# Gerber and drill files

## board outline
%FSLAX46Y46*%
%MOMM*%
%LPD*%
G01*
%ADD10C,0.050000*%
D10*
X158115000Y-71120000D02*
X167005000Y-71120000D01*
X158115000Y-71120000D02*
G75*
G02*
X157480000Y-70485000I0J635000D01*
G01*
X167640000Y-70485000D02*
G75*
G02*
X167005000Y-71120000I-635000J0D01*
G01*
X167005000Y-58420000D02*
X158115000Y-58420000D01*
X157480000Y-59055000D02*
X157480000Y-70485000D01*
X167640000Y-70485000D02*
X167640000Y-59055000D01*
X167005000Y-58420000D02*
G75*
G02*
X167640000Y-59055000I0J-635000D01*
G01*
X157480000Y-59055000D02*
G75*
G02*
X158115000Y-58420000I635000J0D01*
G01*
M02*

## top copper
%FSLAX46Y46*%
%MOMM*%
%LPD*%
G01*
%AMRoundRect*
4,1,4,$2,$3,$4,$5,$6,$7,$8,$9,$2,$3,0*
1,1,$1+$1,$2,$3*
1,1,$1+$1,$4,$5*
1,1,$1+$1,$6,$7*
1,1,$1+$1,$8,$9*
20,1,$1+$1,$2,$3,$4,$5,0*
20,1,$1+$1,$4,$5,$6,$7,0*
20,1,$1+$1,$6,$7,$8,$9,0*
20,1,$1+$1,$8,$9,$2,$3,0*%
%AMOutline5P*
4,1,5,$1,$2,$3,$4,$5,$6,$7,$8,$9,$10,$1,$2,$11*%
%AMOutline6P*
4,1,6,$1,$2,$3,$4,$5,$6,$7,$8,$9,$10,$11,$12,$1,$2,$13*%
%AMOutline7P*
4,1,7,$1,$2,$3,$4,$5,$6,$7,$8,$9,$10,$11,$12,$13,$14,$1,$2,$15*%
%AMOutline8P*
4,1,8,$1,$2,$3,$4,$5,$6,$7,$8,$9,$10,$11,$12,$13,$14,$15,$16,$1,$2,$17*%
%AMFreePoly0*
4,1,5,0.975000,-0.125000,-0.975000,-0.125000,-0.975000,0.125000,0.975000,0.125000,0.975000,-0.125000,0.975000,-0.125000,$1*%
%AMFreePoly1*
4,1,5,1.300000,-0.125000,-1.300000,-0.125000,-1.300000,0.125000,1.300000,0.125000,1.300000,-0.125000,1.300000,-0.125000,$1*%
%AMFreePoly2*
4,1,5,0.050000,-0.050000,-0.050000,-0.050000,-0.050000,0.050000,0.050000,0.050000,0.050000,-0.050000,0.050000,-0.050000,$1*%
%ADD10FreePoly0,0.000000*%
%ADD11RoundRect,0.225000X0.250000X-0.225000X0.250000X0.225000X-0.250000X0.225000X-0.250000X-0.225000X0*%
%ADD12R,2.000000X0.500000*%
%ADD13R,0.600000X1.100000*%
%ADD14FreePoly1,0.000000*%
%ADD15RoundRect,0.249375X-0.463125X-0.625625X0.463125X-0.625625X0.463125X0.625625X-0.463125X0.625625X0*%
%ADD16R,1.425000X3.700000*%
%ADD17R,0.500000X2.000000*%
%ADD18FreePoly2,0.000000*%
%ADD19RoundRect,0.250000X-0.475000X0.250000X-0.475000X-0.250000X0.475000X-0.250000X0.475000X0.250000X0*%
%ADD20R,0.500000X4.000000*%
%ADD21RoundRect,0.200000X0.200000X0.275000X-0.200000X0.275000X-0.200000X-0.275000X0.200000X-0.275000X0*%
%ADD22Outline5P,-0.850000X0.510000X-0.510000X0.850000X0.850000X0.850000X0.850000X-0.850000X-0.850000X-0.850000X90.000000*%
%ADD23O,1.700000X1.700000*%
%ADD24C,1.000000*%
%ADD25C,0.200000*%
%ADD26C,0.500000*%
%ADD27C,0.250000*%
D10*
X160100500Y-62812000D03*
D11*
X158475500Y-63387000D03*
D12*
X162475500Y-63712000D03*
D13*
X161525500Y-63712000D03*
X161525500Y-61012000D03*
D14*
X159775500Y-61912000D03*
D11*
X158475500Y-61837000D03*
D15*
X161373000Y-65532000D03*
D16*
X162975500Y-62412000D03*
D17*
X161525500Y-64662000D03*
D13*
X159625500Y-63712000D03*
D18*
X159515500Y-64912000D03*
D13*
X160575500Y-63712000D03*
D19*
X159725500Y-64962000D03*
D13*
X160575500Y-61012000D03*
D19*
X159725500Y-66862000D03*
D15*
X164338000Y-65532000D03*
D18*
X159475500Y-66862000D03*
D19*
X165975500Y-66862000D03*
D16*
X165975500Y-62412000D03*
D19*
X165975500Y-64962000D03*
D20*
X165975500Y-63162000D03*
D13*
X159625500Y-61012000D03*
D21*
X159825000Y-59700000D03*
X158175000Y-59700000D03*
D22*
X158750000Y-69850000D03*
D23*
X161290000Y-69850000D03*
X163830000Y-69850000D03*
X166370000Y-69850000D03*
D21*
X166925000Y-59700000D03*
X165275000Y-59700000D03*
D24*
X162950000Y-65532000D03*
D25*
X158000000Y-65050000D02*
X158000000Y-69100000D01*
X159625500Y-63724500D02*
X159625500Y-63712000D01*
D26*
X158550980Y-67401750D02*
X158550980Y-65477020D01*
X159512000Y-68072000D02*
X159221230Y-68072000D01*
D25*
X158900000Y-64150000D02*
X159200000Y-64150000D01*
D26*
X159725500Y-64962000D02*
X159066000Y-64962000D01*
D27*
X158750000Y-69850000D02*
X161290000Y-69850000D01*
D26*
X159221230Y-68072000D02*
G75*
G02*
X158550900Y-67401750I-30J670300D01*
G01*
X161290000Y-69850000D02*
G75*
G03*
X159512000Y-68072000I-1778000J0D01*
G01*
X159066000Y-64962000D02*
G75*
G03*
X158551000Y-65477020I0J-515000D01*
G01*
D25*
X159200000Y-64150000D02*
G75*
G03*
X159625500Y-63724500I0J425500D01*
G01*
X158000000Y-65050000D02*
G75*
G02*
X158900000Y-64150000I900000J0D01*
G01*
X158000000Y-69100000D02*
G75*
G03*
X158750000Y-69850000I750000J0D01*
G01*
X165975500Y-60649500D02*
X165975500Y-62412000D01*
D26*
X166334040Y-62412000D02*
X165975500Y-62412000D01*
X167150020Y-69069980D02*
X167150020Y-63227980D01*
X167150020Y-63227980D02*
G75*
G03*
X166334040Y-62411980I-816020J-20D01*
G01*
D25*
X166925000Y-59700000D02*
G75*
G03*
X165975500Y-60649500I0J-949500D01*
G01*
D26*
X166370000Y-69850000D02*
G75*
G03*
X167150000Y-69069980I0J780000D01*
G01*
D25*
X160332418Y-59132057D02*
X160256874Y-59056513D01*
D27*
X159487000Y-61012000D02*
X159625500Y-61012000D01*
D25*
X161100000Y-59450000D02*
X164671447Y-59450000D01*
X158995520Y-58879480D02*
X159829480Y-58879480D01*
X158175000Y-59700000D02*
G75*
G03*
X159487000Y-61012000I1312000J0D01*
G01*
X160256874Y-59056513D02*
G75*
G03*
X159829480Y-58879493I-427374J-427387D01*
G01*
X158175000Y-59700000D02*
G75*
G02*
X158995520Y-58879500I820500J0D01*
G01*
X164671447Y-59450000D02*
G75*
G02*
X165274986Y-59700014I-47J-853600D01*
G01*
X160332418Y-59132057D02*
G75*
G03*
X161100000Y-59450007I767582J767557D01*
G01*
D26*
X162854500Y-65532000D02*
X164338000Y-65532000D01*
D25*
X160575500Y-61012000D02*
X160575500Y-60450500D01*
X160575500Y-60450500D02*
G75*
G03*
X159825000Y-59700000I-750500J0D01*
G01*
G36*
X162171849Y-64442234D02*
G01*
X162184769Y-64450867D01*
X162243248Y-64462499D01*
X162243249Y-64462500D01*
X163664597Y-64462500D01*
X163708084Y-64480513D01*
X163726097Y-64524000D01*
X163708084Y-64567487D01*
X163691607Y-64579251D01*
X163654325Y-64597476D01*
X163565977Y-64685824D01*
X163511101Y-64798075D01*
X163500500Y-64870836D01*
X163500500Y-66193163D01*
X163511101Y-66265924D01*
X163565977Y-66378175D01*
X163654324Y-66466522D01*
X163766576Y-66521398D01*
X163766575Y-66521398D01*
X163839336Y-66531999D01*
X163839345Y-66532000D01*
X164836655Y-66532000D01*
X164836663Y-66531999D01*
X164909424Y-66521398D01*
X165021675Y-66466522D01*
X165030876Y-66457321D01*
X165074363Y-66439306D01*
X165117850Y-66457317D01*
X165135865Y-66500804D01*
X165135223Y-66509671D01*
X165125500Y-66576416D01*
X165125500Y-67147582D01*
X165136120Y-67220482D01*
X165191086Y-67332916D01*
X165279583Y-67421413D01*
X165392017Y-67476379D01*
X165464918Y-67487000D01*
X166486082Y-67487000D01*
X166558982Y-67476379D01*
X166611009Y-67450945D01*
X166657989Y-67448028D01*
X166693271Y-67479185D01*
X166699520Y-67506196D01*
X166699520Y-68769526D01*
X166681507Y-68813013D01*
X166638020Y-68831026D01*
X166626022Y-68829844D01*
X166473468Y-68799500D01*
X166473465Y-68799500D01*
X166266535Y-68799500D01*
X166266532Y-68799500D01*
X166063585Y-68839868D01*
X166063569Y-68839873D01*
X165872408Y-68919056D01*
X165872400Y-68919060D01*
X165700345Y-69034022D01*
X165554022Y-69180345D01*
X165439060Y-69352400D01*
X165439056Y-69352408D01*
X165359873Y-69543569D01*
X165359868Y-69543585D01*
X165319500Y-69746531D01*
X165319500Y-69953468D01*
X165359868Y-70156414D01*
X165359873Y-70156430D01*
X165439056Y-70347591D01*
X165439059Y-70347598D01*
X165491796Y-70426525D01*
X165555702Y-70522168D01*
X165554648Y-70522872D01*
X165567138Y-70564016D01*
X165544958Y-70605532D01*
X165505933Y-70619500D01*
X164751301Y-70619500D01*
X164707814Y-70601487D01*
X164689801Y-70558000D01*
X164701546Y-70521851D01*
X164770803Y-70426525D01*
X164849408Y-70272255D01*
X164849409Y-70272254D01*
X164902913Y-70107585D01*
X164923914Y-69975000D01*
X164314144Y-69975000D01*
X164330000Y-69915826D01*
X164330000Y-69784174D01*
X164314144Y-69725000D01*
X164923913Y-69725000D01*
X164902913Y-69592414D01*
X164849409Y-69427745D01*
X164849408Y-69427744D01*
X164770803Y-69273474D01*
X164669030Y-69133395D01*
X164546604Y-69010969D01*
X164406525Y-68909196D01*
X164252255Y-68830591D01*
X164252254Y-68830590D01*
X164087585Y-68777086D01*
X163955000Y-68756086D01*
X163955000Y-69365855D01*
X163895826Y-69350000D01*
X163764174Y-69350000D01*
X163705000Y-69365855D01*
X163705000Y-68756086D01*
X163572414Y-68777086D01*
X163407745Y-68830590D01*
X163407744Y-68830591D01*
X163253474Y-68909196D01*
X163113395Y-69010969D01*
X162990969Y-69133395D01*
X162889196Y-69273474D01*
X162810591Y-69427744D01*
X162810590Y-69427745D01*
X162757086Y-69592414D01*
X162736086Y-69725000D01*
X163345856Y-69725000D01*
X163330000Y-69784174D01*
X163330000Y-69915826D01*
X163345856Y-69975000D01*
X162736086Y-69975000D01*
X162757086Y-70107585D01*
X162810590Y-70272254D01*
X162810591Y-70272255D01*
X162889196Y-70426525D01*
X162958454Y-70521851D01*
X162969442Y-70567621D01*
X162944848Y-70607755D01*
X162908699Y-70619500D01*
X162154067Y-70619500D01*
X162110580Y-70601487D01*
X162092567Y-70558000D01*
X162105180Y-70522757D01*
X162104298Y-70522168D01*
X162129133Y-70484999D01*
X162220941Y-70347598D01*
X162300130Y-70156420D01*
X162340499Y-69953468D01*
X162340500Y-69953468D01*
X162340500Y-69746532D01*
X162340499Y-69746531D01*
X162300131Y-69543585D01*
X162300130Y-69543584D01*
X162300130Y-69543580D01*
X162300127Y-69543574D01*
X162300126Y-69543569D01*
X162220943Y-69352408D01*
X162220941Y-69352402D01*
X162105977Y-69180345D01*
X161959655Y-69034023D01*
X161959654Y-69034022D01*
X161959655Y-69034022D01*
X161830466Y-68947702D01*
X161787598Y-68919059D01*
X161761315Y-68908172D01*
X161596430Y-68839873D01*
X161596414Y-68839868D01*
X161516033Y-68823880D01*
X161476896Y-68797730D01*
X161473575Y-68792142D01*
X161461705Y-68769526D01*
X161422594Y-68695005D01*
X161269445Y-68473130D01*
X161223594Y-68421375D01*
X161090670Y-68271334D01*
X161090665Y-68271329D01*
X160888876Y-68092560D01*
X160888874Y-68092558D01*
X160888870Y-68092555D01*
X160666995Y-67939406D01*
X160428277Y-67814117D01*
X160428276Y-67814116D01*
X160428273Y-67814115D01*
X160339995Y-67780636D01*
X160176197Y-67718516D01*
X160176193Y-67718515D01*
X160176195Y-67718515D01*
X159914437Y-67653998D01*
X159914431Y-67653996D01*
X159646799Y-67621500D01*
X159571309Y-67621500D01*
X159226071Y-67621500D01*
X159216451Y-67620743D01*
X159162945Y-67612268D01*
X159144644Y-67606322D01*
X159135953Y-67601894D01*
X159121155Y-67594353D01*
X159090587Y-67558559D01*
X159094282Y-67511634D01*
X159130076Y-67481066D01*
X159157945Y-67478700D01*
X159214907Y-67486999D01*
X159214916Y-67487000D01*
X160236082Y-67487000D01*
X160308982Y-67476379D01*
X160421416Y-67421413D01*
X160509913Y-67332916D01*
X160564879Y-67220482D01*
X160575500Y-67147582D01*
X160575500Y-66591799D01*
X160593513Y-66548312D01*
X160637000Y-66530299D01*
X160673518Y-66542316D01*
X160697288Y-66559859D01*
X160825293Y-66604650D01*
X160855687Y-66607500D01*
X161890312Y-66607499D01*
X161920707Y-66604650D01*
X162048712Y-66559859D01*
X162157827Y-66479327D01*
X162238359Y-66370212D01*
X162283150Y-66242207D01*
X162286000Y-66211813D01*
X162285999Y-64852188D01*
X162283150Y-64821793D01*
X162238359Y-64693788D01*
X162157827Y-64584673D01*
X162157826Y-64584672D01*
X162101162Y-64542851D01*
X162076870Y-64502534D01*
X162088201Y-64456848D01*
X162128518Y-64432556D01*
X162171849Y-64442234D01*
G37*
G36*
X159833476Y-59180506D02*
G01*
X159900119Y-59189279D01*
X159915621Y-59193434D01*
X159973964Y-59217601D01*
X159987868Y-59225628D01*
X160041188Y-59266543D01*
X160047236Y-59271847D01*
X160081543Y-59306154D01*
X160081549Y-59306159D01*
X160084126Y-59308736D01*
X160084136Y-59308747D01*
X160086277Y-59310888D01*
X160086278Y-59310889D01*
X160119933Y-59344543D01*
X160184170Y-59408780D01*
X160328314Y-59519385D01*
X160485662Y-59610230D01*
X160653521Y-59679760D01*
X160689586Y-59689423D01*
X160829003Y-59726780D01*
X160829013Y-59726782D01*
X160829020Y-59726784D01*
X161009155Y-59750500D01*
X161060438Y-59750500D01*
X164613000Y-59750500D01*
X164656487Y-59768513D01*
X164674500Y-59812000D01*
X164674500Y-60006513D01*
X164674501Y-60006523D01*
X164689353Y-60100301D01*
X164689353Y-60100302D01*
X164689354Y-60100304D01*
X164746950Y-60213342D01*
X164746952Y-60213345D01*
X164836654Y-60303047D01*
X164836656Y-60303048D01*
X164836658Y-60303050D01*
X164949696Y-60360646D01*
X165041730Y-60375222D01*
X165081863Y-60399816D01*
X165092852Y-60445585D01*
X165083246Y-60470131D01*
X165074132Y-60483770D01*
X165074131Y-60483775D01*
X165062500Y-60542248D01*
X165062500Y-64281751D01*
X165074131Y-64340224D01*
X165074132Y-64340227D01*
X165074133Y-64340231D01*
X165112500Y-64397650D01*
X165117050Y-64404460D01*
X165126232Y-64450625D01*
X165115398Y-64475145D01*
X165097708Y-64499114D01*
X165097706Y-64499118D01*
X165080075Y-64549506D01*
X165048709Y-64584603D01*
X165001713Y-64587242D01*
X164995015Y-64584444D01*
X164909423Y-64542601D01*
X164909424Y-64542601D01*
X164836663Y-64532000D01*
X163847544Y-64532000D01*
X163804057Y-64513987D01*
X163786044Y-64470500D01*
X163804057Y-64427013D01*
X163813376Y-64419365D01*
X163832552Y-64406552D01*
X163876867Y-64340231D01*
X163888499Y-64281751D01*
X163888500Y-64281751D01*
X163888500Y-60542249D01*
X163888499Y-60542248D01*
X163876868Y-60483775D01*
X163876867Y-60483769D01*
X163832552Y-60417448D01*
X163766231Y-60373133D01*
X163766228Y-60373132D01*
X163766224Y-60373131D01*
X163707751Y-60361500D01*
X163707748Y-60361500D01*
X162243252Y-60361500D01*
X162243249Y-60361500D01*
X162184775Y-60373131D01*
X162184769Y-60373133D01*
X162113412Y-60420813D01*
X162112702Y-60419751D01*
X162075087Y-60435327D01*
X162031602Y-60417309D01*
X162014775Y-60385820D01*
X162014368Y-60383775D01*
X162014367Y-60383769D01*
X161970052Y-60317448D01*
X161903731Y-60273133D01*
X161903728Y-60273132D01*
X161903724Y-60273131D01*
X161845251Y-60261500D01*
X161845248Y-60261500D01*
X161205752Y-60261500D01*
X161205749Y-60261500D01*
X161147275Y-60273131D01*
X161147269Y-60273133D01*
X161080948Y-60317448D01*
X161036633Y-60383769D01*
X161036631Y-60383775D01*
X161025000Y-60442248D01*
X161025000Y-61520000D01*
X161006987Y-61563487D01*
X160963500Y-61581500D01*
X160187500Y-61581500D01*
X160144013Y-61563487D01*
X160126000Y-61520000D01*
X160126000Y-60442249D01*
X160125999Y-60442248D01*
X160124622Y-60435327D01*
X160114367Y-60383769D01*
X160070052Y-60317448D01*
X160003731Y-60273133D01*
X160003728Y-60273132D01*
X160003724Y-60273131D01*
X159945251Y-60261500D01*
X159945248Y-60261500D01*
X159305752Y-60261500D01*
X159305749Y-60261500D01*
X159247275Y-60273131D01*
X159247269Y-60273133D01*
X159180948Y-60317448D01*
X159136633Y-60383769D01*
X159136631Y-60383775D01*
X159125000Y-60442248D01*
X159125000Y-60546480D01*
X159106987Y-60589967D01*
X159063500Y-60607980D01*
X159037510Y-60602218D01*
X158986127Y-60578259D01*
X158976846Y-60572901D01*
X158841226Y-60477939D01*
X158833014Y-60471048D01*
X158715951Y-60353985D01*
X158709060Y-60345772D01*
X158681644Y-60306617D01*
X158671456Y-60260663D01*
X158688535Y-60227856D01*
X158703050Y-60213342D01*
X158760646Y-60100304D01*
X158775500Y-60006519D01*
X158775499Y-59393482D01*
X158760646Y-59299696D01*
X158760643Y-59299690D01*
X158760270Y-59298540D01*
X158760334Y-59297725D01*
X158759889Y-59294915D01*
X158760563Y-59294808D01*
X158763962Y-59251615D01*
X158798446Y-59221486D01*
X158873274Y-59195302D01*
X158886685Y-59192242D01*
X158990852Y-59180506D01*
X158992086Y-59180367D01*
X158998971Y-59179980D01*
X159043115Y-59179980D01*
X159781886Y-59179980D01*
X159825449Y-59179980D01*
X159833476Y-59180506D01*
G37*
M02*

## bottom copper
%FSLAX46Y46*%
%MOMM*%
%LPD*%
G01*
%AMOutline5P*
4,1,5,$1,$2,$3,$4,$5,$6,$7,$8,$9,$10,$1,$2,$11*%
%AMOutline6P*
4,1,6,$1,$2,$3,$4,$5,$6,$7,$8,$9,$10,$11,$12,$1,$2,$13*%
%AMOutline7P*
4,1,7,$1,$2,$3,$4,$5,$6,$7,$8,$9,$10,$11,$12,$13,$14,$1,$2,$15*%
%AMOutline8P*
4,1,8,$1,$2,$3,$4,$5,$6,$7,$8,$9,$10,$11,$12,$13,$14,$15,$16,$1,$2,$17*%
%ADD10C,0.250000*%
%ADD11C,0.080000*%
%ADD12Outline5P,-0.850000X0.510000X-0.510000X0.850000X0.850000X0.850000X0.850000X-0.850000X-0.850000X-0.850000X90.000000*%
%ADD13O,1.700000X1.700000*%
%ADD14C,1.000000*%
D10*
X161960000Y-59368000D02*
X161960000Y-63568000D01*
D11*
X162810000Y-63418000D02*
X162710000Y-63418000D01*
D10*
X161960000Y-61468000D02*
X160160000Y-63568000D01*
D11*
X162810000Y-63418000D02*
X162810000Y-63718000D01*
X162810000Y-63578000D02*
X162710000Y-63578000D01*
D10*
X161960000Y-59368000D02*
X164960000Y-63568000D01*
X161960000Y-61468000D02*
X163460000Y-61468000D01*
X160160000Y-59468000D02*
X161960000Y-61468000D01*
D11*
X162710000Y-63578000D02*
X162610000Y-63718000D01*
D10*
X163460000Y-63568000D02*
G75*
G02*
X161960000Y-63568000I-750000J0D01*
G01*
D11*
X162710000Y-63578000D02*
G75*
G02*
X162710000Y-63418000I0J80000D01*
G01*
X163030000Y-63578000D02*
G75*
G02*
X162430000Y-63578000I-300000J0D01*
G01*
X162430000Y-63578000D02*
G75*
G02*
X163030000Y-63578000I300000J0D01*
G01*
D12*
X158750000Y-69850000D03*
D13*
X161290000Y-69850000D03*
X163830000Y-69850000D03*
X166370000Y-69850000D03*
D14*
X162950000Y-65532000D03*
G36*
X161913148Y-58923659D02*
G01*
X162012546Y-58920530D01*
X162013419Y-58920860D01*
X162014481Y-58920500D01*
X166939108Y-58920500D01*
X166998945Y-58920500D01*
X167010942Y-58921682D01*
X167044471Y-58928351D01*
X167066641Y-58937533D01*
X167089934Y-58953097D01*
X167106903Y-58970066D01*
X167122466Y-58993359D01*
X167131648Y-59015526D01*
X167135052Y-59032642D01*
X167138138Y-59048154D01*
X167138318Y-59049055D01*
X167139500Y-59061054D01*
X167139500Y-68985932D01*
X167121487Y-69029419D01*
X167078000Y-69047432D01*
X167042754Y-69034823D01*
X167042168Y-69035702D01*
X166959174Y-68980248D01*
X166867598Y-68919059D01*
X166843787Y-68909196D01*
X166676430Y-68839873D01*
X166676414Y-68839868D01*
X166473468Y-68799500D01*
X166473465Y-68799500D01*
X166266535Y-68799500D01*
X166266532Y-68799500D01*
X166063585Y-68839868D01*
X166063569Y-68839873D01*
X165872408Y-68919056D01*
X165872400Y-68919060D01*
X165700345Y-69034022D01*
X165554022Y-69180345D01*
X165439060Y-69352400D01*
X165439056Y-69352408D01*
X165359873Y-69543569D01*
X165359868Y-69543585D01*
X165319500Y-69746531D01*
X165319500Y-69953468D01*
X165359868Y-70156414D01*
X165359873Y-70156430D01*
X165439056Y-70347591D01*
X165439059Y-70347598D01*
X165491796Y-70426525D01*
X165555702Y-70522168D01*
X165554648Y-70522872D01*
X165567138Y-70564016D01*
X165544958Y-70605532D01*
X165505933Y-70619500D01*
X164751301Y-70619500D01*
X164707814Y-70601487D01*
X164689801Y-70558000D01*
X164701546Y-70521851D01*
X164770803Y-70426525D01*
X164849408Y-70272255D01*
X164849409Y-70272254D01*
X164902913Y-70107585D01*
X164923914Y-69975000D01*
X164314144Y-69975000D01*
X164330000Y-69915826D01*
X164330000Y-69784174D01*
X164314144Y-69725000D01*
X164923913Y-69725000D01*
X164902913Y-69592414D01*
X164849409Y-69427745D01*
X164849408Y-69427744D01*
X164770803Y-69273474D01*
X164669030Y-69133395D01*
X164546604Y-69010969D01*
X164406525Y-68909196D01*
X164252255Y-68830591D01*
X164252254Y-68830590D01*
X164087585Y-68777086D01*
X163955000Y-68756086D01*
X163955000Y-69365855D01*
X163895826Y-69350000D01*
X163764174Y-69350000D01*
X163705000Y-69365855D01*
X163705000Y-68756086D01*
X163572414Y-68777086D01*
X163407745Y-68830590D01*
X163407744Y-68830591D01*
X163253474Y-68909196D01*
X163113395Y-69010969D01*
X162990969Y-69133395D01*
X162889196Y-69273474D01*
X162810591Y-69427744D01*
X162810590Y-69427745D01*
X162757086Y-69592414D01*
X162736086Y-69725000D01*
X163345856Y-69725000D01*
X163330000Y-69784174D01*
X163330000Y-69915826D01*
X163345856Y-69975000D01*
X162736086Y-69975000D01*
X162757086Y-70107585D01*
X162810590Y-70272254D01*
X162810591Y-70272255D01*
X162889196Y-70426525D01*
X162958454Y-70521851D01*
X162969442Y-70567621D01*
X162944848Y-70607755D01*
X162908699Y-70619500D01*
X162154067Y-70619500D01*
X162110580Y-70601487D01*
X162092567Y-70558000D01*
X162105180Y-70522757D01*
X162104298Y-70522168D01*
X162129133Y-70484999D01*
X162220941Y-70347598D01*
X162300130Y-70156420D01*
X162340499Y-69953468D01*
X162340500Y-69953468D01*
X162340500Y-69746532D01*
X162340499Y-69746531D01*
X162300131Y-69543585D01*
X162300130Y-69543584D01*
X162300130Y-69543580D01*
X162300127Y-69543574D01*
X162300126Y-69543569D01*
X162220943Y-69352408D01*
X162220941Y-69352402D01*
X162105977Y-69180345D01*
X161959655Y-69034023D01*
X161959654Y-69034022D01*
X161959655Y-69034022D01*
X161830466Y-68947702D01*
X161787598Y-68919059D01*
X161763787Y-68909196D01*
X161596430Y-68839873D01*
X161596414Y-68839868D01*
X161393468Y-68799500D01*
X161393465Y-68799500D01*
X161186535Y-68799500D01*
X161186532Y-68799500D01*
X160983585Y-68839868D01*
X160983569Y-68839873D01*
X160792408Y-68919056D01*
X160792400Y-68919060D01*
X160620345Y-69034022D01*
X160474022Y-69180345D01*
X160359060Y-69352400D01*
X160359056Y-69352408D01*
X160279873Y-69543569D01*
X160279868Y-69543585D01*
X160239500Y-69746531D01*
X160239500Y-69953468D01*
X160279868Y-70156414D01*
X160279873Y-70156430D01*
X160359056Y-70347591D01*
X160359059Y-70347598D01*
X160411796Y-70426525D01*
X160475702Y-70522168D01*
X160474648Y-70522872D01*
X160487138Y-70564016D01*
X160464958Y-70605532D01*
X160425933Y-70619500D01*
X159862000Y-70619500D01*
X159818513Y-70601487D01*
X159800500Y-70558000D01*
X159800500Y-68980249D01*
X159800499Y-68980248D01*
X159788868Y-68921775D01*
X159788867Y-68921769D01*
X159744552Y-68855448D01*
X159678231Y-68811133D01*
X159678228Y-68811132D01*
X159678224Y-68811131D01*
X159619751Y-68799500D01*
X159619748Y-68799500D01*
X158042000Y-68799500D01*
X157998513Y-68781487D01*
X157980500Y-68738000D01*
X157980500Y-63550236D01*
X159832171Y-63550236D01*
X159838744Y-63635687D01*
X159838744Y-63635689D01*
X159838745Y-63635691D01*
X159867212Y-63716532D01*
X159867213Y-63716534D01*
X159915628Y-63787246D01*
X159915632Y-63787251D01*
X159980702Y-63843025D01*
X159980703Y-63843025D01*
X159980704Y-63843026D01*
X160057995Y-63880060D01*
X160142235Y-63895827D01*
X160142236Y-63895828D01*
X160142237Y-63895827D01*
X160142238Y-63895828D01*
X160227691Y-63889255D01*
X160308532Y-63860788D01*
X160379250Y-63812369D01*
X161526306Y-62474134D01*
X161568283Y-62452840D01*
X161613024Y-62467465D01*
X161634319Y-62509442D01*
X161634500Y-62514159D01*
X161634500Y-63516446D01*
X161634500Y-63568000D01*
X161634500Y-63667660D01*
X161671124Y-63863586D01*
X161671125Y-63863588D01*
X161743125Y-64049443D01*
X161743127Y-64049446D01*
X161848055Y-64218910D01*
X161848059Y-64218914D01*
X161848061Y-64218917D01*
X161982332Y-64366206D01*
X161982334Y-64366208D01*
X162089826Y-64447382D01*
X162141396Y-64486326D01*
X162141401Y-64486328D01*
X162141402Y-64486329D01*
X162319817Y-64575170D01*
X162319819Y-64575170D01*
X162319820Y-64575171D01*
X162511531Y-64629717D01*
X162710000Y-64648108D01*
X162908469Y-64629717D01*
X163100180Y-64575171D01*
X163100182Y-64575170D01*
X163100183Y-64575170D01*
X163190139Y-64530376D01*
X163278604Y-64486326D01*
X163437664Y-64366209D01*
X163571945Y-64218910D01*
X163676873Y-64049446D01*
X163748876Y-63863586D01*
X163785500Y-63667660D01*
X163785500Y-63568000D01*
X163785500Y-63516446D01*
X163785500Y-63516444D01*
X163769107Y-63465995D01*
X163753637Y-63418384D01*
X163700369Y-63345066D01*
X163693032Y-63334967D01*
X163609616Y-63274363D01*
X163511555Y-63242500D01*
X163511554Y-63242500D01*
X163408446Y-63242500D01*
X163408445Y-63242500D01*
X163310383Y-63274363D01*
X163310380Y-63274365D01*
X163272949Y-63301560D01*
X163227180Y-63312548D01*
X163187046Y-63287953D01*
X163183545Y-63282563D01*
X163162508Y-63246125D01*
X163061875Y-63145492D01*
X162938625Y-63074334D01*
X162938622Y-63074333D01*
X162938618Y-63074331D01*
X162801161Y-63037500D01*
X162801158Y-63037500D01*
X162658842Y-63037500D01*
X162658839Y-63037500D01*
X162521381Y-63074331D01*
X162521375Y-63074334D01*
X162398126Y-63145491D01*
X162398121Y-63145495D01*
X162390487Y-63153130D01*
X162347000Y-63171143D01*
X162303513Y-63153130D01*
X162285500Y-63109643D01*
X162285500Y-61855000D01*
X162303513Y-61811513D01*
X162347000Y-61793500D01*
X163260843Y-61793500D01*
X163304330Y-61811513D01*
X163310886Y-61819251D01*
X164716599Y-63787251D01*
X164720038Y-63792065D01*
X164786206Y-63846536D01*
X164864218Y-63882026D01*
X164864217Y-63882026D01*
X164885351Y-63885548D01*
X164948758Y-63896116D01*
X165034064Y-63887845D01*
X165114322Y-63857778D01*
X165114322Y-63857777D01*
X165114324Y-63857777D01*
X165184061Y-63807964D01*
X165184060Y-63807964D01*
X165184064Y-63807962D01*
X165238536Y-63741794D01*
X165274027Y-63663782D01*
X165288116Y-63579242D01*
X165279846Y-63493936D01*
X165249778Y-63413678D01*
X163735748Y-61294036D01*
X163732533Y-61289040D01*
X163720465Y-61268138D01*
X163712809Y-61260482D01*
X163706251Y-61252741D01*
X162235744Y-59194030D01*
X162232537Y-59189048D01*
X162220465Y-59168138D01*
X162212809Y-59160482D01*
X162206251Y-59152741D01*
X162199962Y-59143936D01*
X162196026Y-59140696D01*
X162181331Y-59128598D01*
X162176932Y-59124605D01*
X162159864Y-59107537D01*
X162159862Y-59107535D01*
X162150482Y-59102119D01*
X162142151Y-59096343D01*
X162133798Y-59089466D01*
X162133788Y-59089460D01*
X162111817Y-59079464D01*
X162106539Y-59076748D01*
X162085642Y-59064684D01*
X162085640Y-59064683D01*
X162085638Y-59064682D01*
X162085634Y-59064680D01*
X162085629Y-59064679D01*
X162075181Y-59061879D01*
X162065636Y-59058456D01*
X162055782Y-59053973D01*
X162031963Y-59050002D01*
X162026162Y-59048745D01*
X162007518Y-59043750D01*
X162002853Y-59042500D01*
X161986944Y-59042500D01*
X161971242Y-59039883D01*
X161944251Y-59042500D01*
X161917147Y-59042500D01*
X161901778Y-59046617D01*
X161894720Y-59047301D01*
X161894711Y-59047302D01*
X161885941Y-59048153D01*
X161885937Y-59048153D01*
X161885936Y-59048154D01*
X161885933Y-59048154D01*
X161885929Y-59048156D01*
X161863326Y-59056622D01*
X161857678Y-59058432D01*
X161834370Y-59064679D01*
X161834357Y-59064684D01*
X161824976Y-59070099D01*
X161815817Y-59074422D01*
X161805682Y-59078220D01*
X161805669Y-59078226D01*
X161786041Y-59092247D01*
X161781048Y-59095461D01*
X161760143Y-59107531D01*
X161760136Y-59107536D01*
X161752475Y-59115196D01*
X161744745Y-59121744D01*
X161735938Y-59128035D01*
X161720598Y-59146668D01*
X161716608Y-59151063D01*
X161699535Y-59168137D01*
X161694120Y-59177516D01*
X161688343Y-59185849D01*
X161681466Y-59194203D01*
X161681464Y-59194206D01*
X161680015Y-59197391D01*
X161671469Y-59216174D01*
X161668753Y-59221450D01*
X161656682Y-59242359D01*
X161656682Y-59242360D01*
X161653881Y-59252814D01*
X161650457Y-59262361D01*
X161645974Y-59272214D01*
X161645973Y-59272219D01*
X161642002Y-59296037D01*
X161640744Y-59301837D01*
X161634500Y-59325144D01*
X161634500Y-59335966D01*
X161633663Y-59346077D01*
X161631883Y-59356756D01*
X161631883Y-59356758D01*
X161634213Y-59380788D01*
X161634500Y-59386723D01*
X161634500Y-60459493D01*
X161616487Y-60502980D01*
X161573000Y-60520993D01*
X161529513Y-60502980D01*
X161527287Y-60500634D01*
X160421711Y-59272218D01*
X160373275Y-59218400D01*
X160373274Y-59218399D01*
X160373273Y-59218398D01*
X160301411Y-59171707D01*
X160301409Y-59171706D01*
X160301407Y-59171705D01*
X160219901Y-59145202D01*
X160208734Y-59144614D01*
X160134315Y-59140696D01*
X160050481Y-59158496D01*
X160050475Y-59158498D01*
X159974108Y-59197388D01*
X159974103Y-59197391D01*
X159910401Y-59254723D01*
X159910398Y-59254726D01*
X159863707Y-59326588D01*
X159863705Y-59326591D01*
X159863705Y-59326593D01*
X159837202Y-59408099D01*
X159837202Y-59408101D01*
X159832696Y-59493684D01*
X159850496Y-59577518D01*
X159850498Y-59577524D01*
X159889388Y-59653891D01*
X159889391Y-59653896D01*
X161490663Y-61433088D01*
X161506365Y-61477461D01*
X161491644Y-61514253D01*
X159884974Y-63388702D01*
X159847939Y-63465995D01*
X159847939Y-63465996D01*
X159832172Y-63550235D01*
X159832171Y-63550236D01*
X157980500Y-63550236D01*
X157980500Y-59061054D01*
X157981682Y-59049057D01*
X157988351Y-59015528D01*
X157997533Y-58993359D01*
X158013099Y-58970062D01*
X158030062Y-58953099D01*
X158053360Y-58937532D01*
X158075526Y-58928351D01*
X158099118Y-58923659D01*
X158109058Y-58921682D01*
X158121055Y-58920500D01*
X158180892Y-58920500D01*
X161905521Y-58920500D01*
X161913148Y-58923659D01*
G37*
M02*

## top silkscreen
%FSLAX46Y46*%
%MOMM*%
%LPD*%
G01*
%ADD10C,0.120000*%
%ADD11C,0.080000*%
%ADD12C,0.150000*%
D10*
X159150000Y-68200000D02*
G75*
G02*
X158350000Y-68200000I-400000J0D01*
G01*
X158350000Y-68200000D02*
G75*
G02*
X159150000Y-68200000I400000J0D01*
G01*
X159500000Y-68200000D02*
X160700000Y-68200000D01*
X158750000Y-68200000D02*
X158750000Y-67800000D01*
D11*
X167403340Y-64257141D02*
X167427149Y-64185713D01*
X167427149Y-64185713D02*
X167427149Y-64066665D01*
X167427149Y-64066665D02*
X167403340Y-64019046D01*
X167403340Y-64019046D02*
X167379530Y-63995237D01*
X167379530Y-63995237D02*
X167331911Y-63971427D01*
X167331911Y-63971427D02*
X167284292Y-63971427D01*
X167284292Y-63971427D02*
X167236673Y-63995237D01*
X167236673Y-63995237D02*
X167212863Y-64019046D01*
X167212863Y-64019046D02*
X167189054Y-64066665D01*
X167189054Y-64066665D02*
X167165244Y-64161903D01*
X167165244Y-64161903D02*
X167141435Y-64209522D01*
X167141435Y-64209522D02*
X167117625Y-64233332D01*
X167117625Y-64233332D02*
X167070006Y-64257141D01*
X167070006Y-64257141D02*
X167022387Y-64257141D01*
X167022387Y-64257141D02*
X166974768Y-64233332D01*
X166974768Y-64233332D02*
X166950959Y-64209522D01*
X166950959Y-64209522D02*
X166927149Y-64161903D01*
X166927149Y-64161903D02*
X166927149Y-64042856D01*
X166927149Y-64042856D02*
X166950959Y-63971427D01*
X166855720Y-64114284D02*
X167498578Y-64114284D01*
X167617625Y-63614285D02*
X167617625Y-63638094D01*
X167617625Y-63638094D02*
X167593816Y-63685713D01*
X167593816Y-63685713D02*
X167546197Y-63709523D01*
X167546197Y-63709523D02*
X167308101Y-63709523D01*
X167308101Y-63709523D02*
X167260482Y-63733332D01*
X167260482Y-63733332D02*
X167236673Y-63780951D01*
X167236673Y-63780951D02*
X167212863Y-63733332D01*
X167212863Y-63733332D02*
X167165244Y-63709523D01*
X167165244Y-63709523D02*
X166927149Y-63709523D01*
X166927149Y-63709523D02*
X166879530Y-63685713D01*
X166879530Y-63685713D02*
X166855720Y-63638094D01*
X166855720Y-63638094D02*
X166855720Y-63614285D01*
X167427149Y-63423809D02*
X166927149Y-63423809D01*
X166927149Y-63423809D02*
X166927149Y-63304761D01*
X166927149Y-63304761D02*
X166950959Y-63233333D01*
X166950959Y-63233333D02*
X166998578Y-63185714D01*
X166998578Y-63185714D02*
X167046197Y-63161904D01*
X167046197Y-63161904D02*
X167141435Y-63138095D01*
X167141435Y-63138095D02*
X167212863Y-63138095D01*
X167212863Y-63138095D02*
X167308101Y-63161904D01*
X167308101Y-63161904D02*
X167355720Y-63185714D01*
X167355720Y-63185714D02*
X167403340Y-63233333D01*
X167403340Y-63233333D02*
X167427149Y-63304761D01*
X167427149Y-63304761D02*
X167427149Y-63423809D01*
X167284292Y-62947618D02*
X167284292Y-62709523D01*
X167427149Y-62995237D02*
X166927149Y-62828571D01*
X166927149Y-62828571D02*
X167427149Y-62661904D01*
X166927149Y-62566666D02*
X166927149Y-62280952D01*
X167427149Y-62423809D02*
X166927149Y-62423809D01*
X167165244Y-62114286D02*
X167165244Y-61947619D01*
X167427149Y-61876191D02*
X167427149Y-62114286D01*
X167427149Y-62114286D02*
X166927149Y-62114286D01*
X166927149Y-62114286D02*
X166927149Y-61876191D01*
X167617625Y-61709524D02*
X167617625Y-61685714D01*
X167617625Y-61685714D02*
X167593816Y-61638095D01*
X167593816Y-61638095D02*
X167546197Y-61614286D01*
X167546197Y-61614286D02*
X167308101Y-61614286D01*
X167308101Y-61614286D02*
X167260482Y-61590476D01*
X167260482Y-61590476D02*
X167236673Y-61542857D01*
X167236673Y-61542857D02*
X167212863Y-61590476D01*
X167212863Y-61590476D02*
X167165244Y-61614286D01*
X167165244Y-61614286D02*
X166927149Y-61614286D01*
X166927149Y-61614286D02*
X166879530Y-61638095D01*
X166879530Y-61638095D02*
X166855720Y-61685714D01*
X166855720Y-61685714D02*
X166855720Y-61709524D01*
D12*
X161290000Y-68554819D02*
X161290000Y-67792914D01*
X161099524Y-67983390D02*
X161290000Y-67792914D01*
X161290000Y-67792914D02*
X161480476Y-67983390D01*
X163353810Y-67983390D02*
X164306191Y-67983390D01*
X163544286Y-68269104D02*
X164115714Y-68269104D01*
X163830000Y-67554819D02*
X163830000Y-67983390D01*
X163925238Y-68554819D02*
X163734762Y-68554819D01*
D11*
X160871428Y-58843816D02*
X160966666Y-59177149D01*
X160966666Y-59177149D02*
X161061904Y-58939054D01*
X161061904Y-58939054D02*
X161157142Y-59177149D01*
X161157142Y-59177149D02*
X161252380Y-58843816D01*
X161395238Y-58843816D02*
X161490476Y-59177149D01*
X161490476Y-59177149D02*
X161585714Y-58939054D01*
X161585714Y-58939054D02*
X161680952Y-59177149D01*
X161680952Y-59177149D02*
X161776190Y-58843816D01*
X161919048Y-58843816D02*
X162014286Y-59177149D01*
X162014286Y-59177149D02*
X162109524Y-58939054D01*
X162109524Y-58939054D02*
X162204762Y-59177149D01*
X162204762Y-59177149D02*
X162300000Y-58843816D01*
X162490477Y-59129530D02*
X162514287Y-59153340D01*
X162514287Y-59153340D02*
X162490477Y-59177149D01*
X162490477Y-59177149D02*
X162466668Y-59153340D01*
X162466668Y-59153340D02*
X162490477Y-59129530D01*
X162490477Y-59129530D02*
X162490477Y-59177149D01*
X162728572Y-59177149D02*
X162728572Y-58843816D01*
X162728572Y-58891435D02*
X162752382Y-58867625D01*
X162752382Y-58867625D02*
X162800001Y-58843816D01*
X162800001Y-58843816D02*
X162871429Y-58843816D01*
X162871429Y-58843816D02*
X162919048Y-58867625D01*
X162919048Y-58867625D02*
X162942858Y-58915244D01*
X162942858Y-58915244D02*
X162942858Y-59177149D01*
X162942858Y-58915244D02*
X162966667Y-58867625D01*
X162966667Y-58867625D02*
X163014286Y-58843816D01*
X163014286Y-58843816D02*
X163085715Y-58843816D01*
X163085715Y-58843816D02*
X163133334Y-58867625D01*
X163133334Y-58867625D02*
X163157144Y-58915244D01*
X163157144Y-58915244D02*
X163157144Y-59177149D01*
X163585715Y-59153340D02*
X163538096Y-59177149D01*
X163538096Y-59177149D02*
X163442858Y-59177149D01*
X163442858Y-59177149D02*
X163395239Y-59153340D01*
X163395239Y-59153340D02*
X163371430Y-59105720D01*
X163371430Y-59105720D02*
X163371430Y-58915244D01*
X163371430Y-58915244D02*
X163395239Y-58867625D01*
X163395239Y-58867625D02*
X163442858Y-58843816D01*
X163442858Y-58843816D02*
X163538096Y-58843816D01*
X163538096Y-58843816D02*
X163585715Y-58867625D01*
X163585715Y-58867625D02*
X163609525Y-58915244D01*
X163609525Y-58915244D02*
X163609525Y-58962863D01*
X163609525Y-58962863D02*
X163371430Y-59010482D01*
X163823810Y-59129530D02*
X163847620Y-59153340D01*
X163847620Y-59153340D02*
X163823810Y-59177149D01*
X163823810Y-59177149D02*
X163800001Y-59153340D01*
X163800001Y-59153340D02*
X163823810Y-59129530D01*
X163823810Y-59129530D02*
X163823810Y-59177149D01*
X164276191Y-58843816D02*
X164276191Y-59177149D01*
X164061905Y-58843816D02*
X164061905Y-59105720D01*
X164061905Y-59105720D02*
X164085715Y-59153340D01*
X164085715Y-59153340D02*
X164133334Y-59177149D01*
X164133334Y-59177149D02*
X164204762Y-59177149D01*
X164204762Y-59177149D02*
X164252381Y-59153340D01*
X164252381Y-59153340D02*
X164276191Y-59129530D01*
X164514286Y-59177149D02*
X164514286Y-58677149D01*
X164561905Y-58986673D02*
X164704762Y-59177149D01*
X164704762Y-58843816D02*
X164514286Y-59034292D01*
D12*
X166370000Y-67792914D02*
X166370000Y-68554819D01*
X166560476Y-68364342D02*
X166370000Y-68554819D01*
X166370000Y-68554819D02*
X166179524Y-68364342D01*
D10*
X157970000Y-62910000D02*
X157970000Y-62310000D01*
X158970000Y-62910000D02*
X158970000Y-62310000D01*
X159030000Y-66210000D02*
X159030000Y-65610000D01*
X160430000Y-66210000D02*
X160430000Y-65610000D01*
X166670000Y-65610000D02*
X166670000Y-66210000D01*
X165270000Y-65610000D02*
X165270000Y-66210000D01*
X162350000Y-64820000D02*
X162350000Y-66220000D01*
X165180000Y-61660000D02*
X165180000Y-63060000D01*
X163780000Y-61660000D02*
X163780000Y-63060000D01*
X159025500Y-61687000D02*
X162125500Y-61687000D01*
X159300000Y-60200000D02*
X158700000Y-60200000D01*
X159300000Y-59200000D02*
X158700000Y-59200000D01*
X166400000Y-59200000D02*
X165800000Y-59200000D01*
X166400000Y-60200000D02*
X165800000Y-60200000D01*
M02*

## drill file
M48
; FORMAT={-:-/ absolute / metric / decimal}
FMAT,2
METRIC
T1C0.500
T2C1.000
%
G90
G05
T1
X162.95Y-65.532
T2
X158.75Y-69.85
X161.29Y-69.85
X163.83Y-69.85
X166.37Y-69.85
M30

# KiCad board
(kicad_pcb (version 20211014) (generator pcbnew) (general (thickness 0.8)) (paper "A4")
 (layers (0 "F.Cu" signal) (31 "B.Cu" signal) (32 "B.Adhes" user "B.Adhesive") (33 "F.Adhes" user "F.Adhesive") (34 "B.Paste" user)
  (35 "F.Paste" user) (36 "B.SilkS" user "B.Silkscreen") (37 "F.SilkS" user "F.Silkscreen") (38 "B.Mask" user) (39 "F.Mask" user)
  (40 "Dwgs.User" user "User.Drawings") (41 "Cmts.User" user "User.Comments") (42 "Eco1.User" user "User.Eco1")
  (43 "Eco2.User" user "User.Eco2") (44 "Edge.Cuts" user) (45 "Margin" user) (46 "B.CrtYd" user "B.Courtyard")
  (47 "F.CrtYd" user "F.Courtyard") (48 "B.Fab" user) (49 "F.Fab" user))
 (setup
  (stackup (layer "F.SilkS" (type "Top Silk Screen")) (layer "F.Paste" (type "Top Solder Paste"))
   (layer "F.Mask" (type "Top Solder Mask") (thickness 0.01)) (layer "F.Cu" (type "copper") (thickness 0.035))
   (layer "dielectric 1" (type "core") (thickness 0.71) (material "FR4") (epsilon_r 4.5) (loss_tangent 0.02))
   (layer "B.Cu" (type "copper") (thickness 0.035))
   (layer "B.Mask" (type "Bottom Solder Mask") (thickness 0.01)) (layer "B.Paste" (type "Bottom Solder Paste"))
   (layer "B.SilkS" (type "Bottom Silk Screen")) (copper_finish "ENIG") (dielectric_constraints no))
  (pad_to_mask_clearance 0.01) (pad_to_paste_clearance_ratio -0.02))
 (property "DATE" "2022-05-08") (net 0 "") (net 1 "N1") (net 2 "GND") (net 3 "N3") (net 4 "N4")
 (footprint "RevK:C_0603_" (layer "F.Cu") (at 158.47 62.61 90)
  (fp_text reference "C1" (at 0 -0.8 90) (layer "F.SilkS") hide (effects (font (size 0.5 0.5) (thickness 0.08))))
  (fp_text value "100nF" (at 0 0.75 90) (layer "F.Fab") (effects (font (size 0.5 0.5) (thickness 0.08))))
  (fp_line (start -0.3 -0.5) (end 0.3 -0.5) (layer "F.SilkS") (width 0.12))
  (fp_line (start -0.3 0.5) (end 0.3 0.5) (layer "F.SilkS") (width 0.12)))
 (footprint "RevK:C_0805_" (layer "F.Cu") (at 159.73 65.91 90)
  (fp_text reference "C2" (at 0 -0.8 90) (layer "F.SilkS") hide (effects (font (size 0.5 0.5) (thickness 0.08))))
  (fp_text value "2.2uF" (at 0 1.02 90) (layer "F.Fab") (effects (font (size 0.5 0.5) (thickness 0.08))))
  (fp_line (start -0.3 -0.7) (end 0.3 -0.7) (layer "F.SilkS") (width 0.12))
  (fp_line (start -0.3 0.7) (end 0.3 0.7) (layer "F.SilkS") (width 0.12)))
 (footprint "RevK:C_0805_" (layer "F.Cu") (at 165.97 65.91 -90)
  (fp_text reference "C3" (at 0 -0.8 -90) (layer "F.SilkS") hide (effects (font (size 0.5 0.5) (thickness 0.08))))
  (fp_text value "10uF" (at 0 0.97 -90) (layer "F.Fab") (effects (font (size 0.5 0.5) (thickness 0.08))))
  (fp_line (start -0.3 -0.7) (end 0.3 -0.7) (layer "F.SilkS") (width 0.12))
  (fp_line (start -0.3 0.7) (end 0.3 0.7) (layer "F.SilkS") (width 0.12)))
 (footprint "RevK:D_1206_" (layer "F.Cu") (at 162.85 65.52)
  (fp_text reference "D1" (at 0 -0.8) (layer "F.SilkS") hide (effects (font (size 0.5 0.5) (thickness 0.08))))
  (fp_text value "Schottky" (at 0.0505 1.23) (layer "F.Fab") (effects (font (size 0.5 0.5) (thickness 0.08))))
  (fp_line (start -0.5 -0.7) (end -0.5 0.7) (layer "F.SilkS") (width 0.12)))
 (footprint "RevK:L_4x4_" (layer "F.Cu") (at 164.48 62.36)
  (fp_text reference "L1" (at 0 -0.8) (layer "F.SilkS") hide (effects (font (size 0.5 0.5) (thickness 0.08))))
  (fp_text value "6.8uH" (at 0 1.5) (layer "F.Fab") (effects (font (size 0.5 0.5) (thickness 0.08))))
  (fp_line (start 0.7 -0.7) (end 0.7 0.7) (layer "F.SilkS") (width 0.12))
  (fp_line (start -0.7 -0.7) (end -0.7 0.7) (layer "F.SilkS") (width 0.12)))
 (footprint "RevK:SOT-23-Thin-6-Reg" (layer "F.Cu") (at 160.5755 62.362)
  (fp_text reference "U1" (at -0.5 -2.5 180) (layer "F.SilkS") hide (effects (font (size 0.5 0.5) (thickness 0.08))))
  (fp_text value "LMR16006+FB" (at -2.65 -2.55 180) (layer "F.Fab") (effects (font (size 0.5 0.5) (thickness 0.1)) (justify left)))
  (fp_line (start -1.55 -0.675) (end 1.55 -0.675) (layer "F.SilkS") (width 0.12))
  (pad "" smd custom (at -0.475 0.45) (size 1.95 0.25) (layers "F.Cu") (clearance 0.2) (options (clearance outline) (anchor rect))
   (primitives))
  (pad "" smd roundrect (at 5.4 -1.1) (size 1.2 1) (layers "F.Paste") (roundrect_rratio 0.25))
  (pad "" smd roundrect (at -2.1 1.025 90) (size 0.9 0.95) (layers "F.Cu" "F.Paste" "F.Mask") (roundrect_rratio 0.25) (clearance 0.2))
  (pad "" smd rect (at 1.9 1.35) (size 2 0.5) (layers "F.Cu") (clearance 0.2))
  (pad "" smd rect (at 0.95 1.35 90) (size 1.1 0.6) (layers "F.Cu" "F.Paste" "F.Mask") (clearance 0.2))
  (pad "" smd roundrect (at 2.4 1.2) (size 1.2 1) (layers "F.Paste") (roundrect_rratio 0.25))
  (pad "" smd rect (at 0.95 -1.35 90) (size 1.1 0.6) (layers "F.Cu" "F.Paste" "F.Mask") (clearance 0.2))
  (pad "" smd roundrect (at 5.4 1.2) (size 1.2 1) (layers "F.Paste") (roundrect_rratio 0.25))
  (pad "" smd custom (at -0.8 -0.45) (size 2.6 0.25) (layers "F.Cu") (clearance 0.2) (options (clearance outline) (anchor rect))
   (primitives))
  (pad "" smd roundrect (at 2.4 -1.1) (size 1.2 1) (layers "F.Paste") (roundrect_rratio 0.25))
  (pad "" smd roundrect (at -2.1 -0.525 90) (size 0.9 0.95) (layers "F.Cu" "F.Paste" "F.Mask") (roundrect_rratio 0.25) (clearance 0.2))
  (pad "" smd roundrect (at 0.7975 3.17) (size 1.425 1.75) (layers "F.Cu" "F.Paste" "F.Mask") (roundrect_rratio 0.175) (clearance 0.2))
  (pad "" smd roundrect (at 2.4 0.05) (size 1.2 1) (layers "F.Paste") (roundrect_rratio 0.25))
  (pad "" smd rect (at 2.4 0.05 90) (size 3.7 1.425) (layers "F.Cu" "F.Mask") (clearance 0.2))
  (pad "" smd roundrect (at 5.4 0.05) (size 1.2 1) (layers "F.Paste") (roundrect_rratio 0.25))
  (pad "" smd rect (at 0.95 2.3 90) (size 2 0.5) (layers "F.Cu") (clearance 0.2))
  (pad "1" smd rect (at -0.95 1.35 90) (size 1.1 0.6) (layers "F.Cu" "F.Paste" "F.Mask") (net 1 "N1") (clearance 0.2))
  (pad "2" smd custom (at -1.06 2.55) (size 0.1 0.1) (layers "F.Cu") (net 1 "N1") (zone_connect 0)
   (options (clearance outline) (anchor rect)) (primitives))
  (pad "2" smd rect (at 0 1.35 90) (size 1.1 0.6) (layers "F.Cu" "F.Paste" "F.Mask") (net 1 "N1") (clearance 0.2) (zone_connect 0))
  (pad "2" smd roundrect (at -0.85 2.6 270) (size 1 1.45) (layers "F.Cu" "F.Paste" "F.Mask") (roundrect_rratio 0.25) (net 1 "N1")
   (clearance 0.2))
  (pad "3" smd rect (at 0 -1.35 90) (size 1.1 0.6) (layers "F.Cu" "F.Paste" "F.Mask") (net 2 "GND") (clearance 0.2))
  (pad "3" smd roundrect (at -0.85 4.5 270) (size 1 1.45) (layers "F.Cu" "F.Paste" "F.Mask") (roundrect_rratio 0.25) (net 2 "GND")
   (zone_connect 0))
  (pad "3" smd roundrect (at 3.7625 3.17) (size 1.425 1.75) (layers "F.Cu" "F.Paste" "F.Mask") (roundrect_rratio 0.175) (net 2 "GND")
   (clearance 0.2) (zone_connect 0))
  (pad "3" smd custom (at -1.1 4.5) (size 0.1 0.1) (layers "F.Cu") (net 2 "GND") (clearance 0.2) (zone_connect 0)
   (options (clearance outline) (anchor rect)) (primitives))
  (pad "3" smd roundrect (at 5.4 4.5 270) (size 1 1.45) (layers "F.Cu" "F.Paste" "F.Mask") (roundrect_rratio 0.25) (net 2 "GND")
   (zone_connect 0))
  (pad "4" smd rect (at 5.4 0.05 90) (size 3.7 1.425) (layers "F.Cu" "F.Mask") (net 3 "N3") (zone_connect 0))
  (pad "4" smd roundrect (at 5.4 2.6 270) (size 1 1.45) (layers "F.Cu" "F.Paste" "F.Mask") (roundrect_rratio 0.25) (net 3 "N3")
   (clearance 0.2) (zone_connect 0))
  (pad "4" smd rect (at 5.4 0.8) (size 0.5 4) (layers "F.Cu") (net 3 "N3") (zone_connect 0))
  (pad "5" smd rect (at -0.95 -1.35 90) (size 1.1 0.6) (layers "F.Cu" "F.Paste" "F.Mask") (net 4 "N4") (clearance 0.2)))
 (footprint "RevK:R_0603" (layer "F.Cu") (at 159 59.7 180)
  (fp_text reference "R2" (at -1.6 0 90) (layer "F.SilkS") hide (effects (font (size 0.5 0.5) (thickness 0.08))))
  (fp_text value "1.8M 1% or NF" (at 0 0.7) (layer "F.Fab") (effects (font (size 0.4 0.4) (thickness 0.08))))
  (fp_line (start -0.3 -0.5) (end 0.3 -0.5) (layer "F.SilkS") (width 0.12))
  (fp_line (start -0.3 0.5) (end 0.3 0.5) (layer "F.SilkS") (width 0.12))
  (pad "1" smd roundrect (at -0.825 0 180) (size 0.8 0.95) (layers "F.Cu" "F.Paste" "F.Mask") (roundrect_rratio 0.25) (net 2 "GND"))
  (pad "2" smd roundrect (at 0.825 0 180) (size 0.8 0.95) (layers "F.Cu" "F.Paste" "F.Mask") (roundrect_rratio 0.25) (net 4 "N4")))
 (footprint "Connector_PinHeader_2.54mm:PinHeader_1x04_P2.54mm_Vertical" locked (layer "F.Cu") (at 158.75 69.85 90)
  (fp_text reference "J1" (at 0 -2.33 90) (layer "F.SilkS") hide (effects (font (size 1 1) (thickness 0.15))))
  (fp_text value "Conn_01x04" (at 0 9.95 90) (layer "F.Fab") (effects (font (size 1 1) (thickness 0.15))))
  (pad "1" thru_hole roundrect locked (at 0 0 90) (size 1.7 1.7) (drill 1) (layers *.Cu *.Mask) (roundrect_rratio 0) (chamfer_ratio 0.2)
   (chamfer top_left) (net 1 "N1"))
  (pad "2" thru_hole oval locked (at 0 2.54 90) (size 1.7 1.7) (drill 1) (layers *.Cu *.Mask) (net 1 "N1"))
  (pad "3" thru_hole oval locked (at 0 5.08 90) (size 1.7 1.7) (drill 1) (layers *.Cu *.Mask) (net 2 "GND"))
  (pad "4" thru_hole oval locked (at 0 7.62 90) (size 1.7 1.7) (drill 1) (layers *.Cu *.Mask) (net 3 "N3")))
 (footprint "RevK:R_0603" (layer "F.Cu") (at 166.1 59.7 180)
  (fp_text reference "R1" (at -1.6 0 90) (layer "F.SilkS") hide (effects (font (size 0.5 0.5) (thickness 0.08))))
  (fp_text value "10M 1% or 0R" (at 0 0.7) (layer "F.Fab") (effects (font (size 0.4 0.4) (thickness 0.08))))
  (fp_line (start -0.3 0.5) (end 0.3 0.5) (layer "F.SilkS") (width 0.12))
  (fp_line (start -0.3 -0.5) (end 0.3 -0.5) (layer "F.SilkS") (width 0.12))
  (pad "1" smd roundrect (at -0.825 0 180) (size 0.8 0.95) (layers "F.Cu" "F.Paste" "F.Mask") (roundrect_rratio 0.25) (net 3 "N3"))
  (pad "2" smd roundrect (at 0.825 0 180) (size 0.8 0.95) (layers "F.Cu" "F.Paste" "F.Mask") (roundrect_rratio 0.25) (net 4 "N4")))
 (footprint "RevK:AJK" (layer "B.Cu") (at 161.96 61.468 180)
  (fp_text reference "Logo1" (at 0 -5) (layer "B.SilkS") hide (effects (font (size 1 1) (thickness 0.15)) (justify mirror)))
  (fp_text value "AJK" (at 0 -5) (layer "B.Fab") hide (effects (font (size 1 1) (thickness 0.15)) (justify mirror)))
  (fp_line (start 0 2.1) (end 0 -2.1) (layer "B.Cu") (width 0.25))
  (fp_line (start -0.85 -1.95) (end -0.75 -1.95) (layer "B.Cu") (width 0.08))
  (fp_line (start 0 0) (end 1.8 -2.1) (layer "B.Cu") (width 0.25))
  (fp_line (start -0.85 -1.95) (end -0.85 -2.25) (layer "B.Cu") (width 0.08))
  (fp_line (start -0.85 -2.11) (end -0.75 -2.11) (layer "B.Cu") (width 0.08))
  (fp_line (start 0 2.1) (end -3 -2.1) (layer "B.Cu") (width 0.25))
  (fp_line (start 0 0) (end -1.5 0) (layer "B.Cu") (width 0.25))
  (fp_line (start 1.8 2) (end 0 0) (layer "B.Cu") (width 0.25))
  (fp_line (start -0.75 -2.11) (end -0.65 -2.25) (layer "B.Cu") (width 0.08))
  (fp_arc (start -1.5 -2.1) (mid -0.75 -2.85) (end 0 -2.1) (layer "B.Cu") (width 0.25))
  (fp_arc (start -0.75 -2.11) (mid -0.67 -2.03) (end -0.75 -1.95) (layer "B.Cu") (width 0.08))
  (fp_circle (center -0.77 -2.11) (end -0.47 -2.11) (layer "B.Cu") (width 0.08) (fill none)))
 (gr_circle (center 158.75 68.2) (end 158.75 68.6) (layer "F.SilkS") (width 0.12) (fill none))
 (gr_line (start 159.5 68.2) (end 160.7 68.2) (layer "F.SilkS") (width 0.12))
 (gr_line (start 158.75 68.2) (end 158.75 67.8) (layer "F.SilkS") (width 0.12))
 (gr_line (start 158.115 71.12) (end 167.005 71.12) (layer "Edge.Cuts") (width 0.05))
 (gr_arc (start 158.115 71.12) (mid 157.665987 70.934013) (end 157.48 70.485) (layer "Edge.Cuts") (width 0.05))
 (gr_arc (start 167.64 70.485) (mid 167.454013 70.934013) (end 167.005 71.12) (layer "Edge.Cuts") (width 0.05))
 (gr_line (start 167.005 58.42) (end 158.115 58.42) (layer "Edge.Cuts") (width 0.05))
 (gr_line (start 157.48 59.055) (end 157.48 70.485) (layer "Edge.Cuts") (width 0.05))
 (gr_line (start 167.64 70.485) (end 167.64 59.055) (layer "Edge.Cuts") (width 0.05))
 (gr_arc (start 167.005 58.42) (mid 167.454013 58.605987) (end 167.64 59.055) (layer "Edge.Cuts") (width 0.05))
 (gr_arc (start 157.48 59.055) (mid 157.665987 58.605987) (end 158.115 58.42) (layer "Edge.Cuts") (width 0.05))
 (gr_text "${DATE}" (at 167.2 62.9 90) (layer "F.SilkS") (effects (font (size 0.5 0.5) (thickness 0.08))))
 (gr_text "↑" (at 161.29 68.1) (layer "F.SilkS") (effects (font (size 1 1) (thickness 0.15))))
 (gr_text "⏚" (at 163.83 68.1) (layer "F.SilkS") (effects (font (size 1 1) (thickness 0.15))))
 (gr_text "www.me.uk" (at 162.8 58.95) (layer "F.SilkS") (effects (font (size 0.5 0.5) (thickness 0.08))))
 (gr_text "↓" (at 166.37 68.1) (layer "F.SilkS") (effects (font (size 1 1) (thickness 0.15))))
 (segment (start 158 65.05) (end 158 69.1) (width 0.2) (layer "F.Cu") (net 1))
 (segment (start 159.6255 63.7245) (end 159.6255 63.712) (width 0.2) (layer "F.Cu") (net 1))
 (segment (start 158.55098 67.40175) (end 158.55098 65.47702) (width 0.5) (layer "F.Cu") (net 1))
 (segment (start 159.512 68.072) (end 159.22123 68.072) (width 0.5) (layer "F.Cu") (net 1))
 (segment (start 158.9 64.15) (end 159.2 64.15) (width 0.2) (layer "F.Cu") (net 1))
 (segment (start 159.7255 64.962) (end 159.066 64.962) (width 0.5) (layer "F.Cu") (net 1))
 (segment (start 158.75 69.85) (end 161.29 69.85) (width 0.25) (layer "F.Cu") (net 1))
 (arc (start 159.22123 68.072) (mid 158.747292 67.875688) (end 158.55098 67.40175) (width 0.5) (layer "F.Cu") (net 1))
 (arc (start 161.29 69.85) (mid 160.769236 68.592764) (end 159.512 68.072) (width 0.5) (layer "F.Cu") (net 1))
 (arc (start 159.066 64.962) (mid 158.701826 65.112846) (end 158.55098 65.47702) (width 0.5) (layer "F.Cu") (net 1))
 (arc (start 159.2 64.15) (mid 159.500874 64.025374) (end 159.6255 63.7245) (width 0.2) (layer "F.Cu") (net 1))
 (arc (start 158 65.05) (mid 158.263604 64.413604) (end 158.9 64.15) (width 0.2) (layer "F.Cu") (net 1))
 (arc (start 158 69.1) (mid 158.21967 69.63033) (end 158.75 69.85) (width 0.2) (layer "F.Cu") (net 1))
 (segment (start 165.9755 60.6495) (end 165.9755 62.412) (width 0.2) (layer "F.Cu") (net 3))
 (segment (start 166.33404 62.412) (end 165.9755 62.412) (width 0.5) (layer "F.Cu") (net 3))
 (segment (start 167.15002 69.06998) (end 167.15002 63.22798) (width 0.5) (layer "F.Cu") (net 3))
 (arc (start 167.15002 63.22798) (mid 166.911025 62.650995) (end 166.33404 62.412) (width 0.5) (layer "F.Cu") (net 3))
 (arc (start 166.925 59.7) (mid 166.253602 59.978102) (end 165.9755 60.6495) (width 0.2) (layer "F.Cu") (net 3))
 (arc (start 166.37 69.85) (mid 166.921557 69.621537) (end 167.15002 69.06998) (width 0.5) (layer "F.Cu") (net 3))
 (segment (start 160.332418 59.132057) (end 160.256874 59.056513) (width 0.2) (layer "F.Cu") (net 4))
 (segment (start 159.487 61.012) (end 159.6255 61.012) (width 0.25) (layer "F.Cu") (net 4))
 (segment (start 161.1 59.45) (end 164.671447 59.45) (width 0.2) (layer "F.Cu") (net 4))
 (segment (start 158.99552 58.87948) (end 159.82948 58.87948) (width 0.2) (layer "F.Cu") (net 4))
 (arc (start 158.175 59.7) (mid 158.559276 60.627724) (end 159.487 61.012) (width 0.2) (layer "F.Cu") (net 4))
 (arc (start 160.256874 59.056513) (mid 160.060784 58.925489) (end 159.82948 58.87948) (width 0.2) (layer "F.Cu") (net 4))
 (arc (start 158.175 59.7) (mid 158.415325 59.119805) (end 158.99552 58.87948) (width 0.2) (layer "F.Cu") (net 4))
 (arc (start 164.671447 59.45) (mid 164.998087 59.514973) (end 165.275 59.7) (width 0.2) (layer "F.Cu") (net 4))
 (arc (start 160.332418 59.132057) (mid 160.684588 59.367369) (end 161.1 59.45) (width 0.2) (layer "F.Cu") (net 4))
 (segment (start 162.8545 65.532) (end 164.338 65.532) (width 0.5) (layer "F.Cu") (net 2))
 (segment (start 160.5755 61.012) (end 160.5755 60.4505) (width 0.2) (layer "F.Cu") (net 2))
 (via (at 162.95 65.532) (size 1) (drill 0.5) (layers "F.Cu" "B.Cu") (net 2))
 (arc (start 160.5755 60.4505) (mid 160.355684 59.919816) (end 159.825 59.7) (width 0.2) (layer "F.Cu") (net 2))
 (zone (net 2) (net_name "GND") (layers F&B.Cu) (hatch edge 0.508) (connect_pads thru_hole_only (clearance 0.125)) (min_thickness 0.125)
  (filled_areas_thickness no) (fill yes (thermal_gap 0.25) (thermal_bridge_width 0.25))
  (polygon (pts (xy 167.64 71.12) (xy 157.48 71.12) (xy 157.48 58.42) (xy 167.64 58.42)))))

